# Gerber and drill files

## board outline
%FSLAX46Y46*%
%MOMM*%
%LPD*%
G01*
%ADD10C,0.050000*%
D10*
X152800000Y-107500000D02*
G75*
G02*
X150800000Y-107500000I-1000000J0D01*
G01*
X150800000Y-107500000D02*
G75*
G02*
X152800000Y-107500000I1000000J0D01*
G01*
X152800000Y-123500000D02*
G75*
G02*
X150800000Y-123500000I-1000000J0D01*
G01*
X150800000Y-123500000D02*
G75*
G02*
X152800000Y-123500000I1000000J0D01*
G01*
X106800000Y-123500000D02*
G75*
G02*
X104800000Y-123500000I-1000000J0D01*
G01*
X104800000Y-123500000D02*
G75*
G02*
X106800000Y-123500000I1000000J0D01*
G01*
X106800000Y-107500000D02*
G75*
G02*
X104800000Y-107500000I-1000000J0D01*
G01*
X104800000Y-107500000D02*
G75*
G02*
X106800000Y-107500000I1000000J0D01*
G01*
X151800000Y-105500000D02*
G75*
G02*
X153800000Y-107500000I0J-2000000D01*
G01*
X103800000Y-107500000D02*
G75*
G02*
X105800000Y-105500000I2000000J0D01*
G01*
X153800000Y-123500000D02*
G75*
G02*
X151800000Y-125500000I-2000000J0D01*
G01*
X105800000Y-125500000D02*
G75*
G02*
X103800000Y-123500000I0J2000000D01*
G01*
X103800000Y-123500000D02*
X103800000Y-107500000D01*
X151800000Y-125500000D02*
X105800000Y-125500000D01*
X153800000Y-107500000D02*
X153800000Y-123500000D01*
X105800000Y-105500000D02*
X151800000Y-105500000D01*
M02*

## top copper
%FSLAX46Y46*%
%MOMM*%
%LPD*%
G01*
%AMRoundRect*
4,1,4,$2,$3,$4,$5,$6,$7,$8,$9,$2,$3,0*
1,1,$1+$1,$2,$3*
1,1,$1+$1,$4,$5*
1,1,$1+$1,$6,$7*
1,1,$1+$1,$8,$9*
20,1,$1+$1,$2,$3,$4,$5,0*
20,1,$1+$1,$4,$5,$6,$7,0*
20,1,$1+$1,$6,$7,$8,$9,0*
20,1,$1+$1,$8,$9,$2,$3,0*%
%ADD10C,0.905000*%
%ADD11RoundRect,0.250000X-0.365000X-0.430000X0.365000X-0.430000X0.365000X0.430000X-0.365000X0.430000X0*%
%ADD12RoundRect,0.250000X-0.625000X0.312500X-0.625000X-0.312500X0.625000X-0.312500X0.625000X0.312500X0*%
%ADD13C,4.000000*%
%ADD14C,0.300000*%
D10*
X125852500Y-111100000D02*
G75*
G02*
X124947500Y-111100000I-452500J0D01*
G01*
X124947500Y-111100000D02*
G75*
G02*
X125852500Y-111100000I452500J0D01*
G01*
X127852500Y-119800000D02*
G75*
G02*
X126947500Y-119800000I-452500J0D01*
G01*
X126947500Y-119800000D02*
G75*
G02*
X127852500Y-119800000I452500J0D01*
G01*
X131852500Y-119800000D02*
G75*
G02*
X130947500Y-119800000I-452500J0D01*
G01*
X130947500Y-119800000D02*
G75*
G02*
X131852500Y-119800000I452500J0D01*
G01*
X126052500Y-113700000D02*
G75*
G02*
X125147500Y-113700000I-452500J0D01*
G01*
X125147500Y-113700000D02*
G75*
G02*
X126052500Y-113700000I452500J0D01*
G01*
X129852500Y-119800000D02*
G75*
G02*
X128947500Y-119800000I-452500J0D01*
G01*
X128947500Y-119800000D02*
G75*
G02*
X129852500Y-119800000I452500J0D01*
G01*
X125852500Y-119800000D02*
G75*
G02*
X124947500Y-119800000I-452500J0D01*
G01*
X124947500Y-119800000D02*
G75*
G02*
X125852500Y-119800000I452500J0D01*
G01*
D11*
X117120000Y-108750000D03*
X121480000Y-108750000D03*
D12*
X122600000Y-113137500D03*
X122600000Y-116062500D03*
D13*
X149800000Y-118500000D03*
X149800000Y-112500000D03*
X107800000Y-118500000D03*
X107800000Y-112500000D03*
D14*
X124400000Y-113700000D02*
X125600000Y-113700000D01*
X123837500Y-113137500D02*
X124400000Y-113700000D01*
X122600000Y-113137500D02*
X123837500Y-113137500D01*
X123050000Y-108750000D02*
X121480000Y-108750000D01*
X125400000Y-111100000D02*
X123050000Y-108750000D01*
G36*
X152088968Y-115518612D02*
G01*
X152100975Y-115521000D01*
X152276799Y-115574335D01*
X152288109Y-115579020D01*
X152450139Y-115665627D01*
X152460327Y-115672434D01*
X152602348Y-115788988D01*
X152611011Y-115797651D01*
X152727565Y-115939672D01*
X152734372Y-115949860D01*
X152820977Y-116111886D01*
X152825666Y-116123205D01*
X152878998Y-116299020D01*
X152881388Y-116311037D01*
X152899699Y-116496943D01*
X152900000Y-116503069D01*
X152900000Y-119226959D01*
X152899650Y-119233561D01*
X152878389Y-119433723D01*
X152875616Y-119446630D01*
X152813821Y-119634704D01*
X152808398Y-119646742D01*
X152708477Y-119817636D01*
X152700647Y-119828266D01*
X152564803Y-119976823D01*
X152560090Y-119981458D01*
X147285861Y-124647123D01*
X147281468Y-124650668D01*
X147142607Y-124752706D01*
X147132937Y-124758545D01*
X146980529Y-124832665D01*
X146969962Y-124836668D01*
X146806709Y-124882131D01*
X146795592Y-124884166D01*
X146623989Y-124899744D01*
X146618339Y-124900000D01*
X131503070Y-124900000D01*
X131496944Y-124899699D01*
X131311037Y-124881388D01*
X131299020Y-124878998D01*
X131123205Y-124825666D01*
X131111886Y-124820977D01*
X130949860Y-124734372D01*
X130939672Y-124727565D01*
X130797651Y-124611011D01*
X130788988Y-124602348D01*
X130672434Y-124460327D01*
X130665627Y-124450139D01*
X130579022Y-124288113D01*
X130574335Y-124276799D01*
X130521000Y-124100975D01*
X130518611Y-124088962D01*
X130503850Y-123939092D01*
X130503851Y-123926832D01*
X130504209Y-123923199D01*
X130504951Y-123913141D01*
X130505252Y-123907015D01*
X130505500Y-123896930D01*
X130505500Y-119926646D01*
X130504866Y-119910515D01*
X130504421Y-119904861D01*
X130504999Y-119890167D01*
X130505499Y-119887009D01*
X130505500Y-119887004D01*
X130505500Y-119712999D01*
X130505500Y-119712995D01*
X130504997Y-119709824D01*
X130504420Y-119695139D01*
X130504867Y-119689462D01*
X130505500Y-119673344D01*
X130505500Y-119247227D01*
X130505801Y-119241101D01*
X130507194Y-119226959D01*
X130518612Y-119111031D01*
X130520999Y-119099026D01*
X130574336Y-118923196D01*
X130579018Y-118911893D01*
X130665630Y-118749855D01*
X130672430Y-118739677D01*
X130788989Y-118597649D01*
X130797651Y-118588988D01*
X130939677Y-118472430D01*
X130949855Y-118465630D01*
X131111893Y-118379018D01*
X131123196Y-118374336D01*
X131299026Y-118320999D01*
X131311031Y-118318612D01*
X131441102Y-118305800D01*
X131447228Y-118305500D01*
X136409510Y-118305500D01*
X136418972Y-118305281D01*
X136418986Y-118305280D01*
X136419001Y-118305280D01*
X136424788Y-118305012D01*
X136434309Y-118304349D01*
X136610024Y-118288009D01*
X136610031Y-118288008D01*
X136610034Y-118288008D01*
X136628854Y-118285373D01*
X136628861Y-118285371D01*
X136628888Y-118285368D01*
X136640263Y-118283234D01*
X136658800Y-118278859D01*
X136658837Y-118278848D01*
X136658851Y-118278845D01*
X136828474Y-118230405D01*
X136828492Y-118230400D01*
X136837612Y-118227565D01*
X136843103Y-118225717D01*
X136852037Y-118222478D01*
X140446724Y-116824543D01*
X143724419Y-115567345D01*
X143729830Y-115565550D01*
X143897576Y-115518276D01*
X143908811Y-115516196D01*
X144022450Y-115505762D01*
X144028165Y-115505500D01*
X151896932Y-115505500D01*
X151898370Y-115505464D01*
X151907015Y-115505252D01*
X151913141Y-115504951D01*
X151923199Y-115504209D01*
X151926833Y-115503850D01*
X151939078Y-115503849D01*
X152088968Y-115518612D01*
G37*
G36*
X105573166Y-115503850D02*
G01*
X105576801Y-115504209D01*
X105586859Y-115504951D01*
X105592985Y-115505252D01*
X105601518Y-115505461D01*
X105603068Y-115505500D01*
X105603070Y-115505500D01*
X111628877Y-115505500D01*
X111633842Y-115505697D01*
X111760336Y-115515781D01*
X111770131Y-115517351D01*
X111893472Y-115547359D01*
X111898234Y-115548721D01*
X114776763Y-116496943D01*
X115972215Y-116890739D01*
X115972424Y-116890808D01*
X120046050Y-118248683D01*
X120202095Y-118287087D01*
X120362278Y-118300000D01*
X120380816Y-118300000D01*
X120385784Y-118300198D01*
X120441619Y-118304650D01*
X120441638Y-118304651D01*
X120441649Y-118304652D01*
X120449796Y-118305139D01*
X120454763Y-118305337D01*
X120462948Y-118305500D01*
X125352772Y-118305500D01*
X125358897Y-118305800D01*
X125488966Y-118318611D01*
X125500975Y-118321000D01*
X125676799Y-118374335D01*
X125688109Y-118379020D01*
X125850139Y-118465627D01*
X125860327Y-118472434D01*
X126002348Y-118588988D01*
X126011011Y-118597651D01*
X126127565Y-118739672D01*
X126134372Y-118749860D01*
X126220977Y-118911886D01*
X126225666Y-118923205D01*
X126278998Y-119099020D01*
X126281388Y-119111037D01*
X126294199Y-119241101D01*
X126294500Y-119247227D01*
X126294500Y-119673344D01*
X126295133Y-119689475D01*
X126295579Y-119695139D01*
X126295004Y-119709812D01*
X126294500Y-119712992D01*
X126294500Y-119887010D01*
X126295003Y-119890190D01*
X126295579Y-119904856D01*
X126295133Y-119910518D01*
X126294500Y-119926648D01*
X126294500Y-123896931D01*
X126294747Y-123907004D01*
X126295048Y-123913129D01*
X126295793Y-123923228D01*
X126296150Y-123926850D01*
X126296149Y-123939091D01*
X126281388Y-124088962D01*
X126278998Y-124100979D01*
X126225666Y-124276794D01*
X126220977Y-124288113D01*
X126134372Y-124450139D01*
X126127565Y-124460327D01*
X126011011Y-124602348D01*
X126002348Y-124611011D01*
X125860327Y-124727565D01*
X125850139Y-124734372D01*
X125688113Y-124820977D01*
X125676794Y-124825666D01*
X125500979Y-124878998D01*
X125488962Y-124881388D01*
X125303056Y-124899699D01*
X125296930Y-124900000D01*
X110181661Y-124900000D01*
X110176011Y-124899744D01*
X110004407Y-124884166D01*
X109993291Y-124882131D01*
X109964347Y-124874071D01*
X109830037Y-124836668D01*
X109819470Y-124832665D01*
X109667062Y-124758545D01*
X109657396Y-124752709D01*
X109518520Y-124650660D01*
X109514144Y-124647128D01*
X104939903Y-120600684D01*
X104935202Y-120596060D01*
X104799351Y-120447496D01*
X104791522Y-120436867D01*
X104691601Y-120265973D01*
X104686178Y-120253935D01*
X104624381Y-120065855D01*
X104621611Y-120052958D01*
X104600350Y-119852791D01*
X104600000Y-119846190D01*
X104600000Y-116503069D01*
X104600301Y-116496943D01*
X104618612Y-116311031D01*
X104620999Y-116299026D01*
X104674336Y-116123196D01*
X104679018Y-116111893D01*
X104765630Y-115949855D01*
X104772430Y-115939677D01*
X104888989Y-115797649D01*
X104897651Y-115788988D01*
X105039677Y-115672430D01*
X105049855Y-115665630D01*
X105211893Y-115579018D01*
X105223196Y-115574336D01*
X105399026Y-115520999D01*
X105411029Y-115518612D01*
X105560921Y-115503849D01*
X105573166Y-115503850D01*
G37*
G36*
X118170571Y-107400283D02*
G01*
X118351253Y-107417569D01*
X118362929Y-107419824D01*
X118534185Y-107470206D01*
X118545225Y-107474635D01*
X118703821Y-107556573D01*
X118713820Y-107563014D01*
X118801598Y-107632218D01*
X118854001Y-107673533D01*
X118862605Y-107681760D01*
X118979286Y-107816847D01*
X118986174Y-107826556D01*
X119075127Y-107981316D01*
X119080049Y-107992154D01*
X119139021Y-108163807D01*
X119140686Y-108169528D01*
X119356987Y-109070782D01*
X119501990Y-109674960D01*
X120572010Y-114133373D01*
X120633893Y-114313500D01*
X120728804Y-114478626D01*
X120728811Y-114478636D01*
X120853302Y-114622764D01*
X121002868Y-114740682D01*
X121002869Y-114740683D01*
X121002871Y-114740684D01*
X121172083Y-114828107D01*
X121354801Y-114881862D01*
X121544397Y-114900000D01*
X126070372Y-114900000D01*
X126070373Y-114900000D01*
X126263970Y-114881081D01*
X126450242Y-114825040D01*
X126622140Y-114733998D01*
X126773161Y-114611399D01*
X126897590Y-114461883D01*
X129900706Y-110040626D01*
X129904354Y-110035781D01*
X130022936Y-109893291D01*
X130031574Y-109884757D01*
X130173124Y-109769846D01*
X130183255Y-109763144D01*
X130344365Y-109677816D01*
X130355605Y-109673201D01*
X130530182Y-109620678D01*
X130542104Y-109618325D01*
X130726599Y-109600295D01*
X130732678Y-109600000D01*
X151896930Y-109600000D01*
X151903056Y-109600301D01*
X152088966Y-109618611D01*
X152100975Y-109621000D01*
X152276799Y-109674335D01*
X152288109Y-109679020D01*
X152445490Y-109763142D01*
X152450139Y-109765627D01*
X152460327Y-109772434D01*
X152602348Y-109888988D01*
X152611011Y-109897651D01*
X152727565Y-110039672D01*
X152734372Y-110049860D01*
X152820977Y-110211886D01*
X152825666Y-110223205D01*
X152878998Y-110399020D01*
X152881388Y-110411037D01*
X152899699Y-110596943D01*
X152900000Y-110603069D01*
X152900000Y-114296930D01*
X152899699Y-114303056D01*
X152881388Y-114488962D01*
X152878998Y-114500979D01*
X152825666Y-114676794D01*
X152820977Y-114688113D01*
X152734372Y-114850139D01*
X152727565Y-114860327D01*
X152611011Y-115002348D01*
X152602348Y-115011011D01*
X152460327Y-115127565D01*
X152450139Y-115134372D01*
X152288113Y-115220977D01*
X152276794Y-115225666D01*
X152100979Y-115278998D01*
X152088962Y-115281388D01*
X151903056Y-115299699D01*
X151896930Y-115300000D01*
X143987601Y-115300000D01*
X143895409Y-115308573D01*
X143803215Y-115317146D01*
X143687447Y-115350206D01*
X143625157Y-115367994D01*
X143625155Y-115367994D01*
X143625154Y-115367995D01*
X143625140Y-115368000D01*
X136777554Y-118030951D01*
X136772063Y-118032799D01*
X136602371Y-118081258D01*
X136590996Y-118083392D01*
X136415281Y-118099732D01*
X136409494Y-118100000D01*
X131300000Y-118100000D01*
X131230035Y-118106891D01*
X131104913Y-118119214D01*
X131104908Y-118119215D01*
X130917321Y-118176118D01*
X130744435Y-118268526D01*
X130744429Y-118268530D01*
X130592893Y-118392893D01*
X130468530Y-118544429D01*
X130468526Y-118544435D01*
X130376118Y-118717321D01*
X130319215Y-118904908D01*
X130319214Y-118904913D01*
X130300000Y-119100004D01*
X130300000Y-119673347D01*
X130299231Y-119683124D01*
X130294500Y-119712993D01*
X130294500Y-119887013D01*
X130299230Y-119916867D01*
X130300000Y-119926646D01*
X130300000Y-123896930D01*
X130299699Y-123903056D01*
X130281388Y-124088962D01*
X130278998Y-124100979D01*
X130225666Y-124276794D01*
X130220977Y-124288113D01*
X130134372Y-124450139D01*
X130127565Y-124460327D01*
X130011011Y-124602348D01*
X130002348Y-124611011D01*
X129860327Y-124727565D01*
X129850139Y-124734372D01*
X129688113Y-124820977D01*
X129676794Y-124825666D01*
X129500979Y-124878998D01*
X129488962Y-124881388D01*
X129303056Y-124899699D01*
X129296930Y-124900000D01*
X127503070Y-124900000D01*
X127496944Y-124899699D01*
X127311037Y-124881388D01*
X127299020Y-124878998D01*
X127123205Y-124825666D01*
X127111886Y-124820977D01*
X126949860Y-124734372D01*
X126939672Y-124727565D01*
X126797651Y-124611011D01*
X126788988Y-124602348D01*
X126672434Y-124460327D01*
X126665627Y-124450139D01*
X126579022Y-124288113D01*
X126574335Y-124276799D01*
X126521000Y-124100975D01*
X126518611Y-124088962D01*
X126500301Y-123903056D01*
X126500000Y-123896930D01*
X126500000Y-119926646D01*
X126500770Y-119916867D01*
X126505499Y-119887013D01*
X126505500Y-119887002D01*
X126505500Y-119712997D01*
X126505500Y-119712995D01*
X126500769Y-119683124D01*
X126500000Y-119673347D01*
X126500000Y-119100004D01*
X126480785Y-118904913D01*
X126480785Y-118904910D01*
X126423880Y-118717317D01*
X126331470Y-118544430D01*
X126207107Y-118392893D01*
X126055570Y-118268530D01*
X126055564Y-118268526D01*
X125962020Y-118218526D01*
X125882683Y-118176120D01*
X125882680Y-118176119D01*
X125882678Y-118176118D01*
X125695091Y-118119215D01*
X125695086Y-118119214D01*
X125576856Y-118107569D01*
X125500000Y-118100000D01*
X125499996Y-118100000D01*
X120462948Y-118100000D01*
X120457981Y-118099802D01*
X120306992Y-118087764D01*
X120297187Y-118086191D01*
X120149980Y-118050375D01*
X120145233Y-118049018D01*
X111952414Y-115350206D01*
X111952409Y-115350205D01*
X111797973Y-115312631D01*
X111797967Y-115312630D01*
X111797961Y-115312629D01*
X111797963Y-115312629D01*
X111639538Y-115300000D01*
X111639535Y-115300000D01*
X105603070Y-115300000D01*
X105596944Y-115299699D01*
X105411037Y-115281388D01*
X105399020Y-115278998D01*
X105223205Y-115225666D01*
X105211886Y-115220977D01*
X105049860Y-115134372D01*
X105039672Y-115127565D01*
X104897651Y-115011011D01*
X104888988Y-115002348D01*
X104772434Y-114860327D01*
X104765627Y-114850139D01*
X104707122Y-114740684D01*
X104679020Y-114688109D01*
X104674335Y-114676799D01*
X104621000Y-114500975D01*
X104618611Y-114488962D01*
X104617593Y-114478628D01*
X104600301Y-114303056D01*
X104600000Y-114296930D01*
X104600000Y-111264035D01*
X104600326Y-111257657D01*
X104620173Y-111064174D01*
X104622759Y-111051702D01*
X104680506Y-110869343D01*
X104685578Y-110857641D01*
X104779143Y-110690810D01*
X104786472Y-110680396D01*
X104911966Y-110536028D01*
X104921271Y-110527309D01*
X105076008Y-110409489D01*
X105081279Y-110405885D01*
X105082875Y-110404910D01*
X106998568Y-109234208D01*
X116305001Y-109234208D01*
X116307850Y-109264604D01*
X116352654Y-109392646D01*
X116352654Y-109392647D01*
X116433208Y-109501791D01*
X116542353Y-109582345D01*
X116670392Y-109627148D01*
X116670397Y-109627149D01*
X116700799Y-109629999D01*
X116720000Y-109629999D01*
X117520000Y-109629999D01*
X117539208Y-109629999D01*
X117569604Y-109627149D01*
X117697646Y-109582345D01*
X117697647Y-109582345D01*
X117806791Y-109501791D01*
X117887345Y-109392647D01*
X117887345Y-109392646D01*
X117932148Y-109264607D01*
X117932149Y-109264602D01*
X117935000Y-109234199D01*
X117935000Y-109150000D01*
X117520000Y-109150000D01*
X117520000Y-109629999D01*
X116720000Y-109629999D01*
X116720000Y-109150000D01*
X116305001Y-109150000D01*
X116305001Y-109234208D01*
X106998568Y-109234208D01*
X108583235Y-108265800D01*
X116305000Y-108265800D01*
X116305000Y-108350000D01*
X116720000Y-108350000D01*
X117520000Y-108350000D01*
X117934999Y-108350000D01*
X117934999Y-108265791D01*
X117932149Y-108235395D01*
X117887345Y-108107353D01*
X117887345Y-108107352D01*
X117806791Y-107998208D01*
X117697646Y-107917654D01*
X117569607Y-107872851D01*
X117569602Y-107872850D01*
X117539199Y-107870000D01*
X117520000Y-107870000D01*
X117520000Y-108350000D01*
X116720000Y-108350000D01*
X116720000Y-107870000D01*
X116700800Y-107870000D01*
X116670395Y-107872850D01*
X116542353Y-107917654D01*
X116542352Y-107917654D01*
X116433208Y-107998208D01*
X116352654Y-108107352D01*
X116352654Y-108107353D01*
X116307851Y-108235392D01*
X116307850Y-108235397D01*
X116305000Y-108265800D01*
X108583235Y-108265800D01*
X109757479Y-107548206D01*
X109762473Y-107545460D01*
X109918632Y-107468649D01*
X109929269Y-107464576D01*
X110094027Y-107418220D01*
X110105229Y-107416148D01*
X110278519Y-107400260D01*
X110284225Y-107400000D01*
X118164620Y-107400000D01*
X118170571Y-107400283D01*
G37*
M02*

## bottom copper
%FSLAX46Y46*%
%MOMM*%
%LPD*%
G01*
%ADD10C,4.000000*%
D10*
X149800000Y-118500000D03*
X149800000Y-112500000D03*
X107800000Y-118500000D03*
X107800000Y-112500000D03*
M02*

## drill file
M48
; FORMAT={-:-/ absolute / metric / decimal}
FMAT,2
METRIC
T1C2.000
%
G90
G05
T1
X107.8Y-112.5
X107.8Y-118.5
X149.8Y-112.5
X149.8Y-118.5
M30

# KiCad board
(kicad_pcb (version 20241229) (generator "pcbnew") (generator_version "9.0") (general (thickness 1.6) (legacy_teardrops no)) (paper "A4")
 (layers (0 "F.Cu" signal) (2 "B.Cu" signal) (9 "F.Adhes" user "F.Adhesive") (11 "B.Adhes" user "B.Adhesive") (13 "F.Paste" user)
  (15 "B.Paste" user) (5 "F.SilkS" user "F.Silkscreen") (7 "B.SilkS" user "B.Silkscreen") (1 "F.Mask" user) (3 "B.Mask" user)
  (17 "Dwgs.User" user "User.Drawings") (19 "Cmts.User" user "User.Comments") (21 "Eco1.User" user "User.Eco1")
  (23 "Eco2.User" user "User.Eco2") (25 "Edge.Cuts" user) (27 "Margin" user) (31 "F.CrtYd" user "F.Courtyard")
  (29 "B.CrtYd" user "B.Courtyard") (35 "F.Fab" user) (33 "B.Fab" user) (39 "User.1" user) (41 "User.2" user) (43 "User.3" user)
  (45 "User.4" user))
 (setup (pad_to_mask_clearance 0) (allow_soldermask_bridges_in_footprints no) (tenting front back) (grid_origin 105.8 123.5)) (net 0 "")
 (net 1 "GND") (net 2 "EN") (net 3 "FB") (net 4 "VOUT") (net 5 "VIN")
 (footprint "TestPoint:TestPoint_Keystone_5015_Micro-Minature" (layer "F.Cu") (at 131.4 119.8)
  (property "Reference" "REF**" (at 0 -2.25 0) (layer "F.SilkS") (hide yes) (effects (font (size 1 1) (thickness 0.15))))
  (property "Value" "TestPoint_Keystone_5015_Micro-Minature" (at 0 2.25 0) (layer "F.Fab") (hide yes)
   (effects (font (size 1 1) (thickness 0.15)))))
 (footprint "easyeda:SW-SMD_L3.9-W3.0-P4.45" (layer "F.Cu") (at 119.3 108.75)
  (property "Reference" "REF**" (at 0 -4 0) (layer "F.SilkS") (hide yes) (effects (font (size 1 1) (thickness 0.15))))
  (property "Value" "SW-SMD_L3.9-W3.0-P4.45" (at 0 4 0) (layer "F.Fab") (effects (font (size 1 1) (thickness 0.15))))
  (pad "1" smd roundrect (at -2.18 0) (size 1.23 1.36) (layers "F.Cu" "F.Mask" "F.Paste") (roundrect_rratio 0.2032520325) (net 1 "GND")
   (zone_connect 1) (thermal_bridge_width 0.8) (thermal_gap 0.2))
  (pad "2" smd roundrect (at 2.18 0) (size 1.23 1.36) (layers "F.Cu" "F.Mask" "F.Paste") (roundrect_rratio 0.2032520325) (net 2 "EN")))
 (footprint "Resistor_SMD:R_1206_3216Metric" (layer "F.Cu") (at 122.6 114.6 -90)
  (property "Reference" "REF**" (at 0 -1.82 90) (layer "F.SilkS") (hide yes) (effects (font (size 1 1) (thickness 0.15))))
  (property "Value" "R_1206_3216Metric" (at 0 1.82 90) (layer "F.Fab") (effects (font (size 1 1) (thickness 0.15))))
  (pad "1" smd roundrect (at -1.4625 0 270) (size 1.125 1.75) (layers "F.Cu" "F.Mask" "F.Paste") (roundrect_rratio 0.222222) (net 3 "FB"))
  (pad "2" smd roundrect (at 1.4625 0 270) (size 1.125 1.75) (layers "F.Cu" "F.Mask" "F.Paste") (roundrect_rratio 0.222222) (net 1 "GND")))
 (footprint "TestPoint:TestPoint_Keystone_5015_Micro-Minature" (layer "F.Cu") (at 125.4 119.8)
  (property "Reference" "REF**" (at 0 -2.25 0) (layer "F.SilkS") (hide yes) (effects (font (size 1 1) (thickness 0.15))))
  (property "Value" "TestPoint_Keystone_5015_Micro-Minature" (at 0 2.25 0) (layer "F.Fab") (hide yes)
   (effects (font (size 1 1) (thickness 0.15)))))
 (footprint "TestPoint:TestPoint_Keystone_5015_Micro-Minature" (layer "F.Cu") (at 128.5 115.5)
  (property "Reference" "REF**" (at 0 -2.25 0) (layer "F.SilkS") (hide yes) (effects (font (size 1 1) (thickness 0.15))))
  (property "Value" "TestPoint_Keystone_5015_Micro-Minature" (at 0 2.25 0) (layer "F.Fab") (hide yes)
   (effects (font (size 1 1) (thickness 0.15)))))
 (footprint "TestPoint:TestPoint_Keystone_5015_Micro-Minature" (layer "F.Cu") (at 125.6 113.7)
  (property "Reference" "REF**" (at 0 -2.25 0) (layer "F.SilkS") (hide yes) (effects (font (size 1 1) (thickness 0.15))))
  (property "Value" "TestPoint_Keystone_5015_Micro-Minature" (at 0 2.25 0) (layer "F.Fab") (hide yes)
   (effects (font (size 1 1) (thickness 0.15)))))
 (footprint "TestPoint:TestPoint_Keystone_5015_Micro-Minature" (layer "F.Cu") (at 125.4 111.1)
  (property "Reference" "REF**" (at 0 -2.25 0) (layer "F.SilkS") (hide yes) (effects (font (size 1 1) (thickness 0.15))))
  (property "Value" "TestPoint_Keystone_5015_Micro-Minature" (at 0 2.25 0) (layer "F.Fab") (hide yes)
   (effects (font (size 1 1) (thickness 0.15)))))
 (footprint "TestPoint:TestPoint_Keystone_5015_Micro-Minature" (layer "F.Cu") (at 129.4 119.8)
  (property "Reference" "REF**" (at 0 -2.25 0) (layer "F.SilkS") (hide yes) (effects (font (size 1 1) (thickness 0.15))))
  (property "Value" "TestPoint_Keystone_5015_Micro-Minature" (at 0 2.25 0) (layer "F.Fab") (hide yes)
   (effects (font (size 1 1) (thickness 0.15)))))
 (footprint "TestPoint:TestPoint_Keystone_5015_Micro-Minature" (layer "F.Cu") (at 127.4 119.8)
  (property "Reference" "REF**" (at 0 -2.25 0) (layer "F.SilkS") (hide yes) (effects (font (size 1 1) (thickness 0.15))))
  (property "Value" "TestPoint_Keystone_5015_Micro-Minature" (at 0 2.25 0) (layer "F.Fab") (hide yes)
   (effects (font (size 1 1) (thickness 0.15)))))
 (gr_circle (center 125.4 111.1) (end 126.3 111.1) (stroke (width 0.01) (type default)) (fill yes) (layer "F.Cu") (net 2))
 (gr_circle (center 127.4 119.8) (end 128.3 119.8) (stroke (width 0.01) (type default)) (fill yes) (layer "F.Cu") (net 1))
 (gr_circle (center 131.4 119.8) (end 132.3 119.8) (stroke (width 0.01) (type default)) (fill yes) (layer "F.Cu") (net 4))
 (gr_circle (center 125.6 113.7) (end 126.5 113.7) (stroke (width 0.01) (type solid)) (fill yes) (layer "F.Cu") (net 3))
 (gr_circle (center 129.4 119.8) (end 130.3 119.8) (stroke (width 0.01) (type default)) (fill yes) (layer "F.Cu") (net 1))
 (gr_circle (center 125.4 119.8) (end 126.3 119.8) (stroke (width 0.01) (type default)) (fill yes) (layer "F.Cu") (net 5))
 (gr_circle (center 151.8 123.5) (end 151.8 122.5) (stroke (width 0.05) (type default)) (fill no) (layer "Edge.Cuts"))
 (gr_circle (center 151.8 107.5) (end 151.8 108.5) (stroke (width 0.05) (type default)) (fill no) (layer "Edge.Cuts"))
 (gr_line (start 105.8 105.5) (end 151.8 105.5) (stroke (width 0.05) (type default)) (layer "Edge.Cuts"))
 (gr_line (start 103.8 123.5) (end 103.8 107.5) (stroke (width 0.05) (type default)) (layer "Edge.Cuts"))
 (gr_circle (center 105.8 123.5) (end 105.8 122.5) (stroke (width 0.05) (type default)) (fill no) (layer "Edge.Cuts"))
 (gr_arc (start 105.8 125.5) (mid 104.385786 124.914214) (end 103.8 123.5) (stroke (width 0.05) (type default)) (layer "Edge.Cuts"))
 (gr_line (start 151.8 125.5) (end 105.8 125.5) (stroke (width 0.05) (type default)) (layer "Edge.Cuts"))
 (gr_arc (start 153.8 123.5) (mid 153.214214 124.914214) (end 151.8 125.5) (stroke (width 0.05) (type default)) (layer "Edge.Cuts"))
 (gr_circle (center 105.8 107.5) (end 105.8 106.5) (stroke (width 0.05) (type default)) (fill no) (layer "Edge.Cuts"))
 (gr_arc (start 103.8 107.5) (mid 104.385786 106.085786) (end 105.8 105.5) (stroke (width 0.05) (type default)) (layer "Edge.Cuts"))
 (gr_line (start 153.8 107.5) (end 153.8 123.5) (stroke (width 0.05) (type default)) (layer "Edge.Cuts"))
 (gr_arc (start 151.8 105.5) (mid 153.214214 106.085786) (end 153.8 107.5) (stroke (width 0.05) (type default)) (layer "Edge.Cuts"))
 (via (at 149.8 118.5) (size 4) (drill 2) (layers "F.Cu" "B.Cu") (tenting none) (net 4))
 (via (at 149.8 112.5) (size 4) (drill 2) (layers "F.Cu" "B.Cu") (tenting none) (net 1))
 (via (at 107.8 112.5) (size 4) (drill 2) (layers "F.Cu" "B.Cu") (tenting none) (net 1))
 (via (at 107.8 118.5) (size 4) (drill 2) (layers "F.Cu" "B.Cu") (tenting none) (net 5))
 (segment (start 125.4 111.1) (end 123.05 108.75) (width 0.3) (layer "F.Cu") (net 2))
 (segment (start 123.05 108.75) (end 121.48 108.75) (width 0.3) (layer "F.Cu") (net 2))
 (segment (start 122.6 113.1375) (end 123.8375 113.1375) (width 0.3) (layer "F.Cu") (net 3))
 (segment (start 124.4 113.7) (end 125.6 113.7) (width 0.3) (layer "F.Cu") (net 3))
 (segment (start 123.8375 113.1375) (end 124.4 113.7) (width 0.3) (layer "F.Cu") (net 3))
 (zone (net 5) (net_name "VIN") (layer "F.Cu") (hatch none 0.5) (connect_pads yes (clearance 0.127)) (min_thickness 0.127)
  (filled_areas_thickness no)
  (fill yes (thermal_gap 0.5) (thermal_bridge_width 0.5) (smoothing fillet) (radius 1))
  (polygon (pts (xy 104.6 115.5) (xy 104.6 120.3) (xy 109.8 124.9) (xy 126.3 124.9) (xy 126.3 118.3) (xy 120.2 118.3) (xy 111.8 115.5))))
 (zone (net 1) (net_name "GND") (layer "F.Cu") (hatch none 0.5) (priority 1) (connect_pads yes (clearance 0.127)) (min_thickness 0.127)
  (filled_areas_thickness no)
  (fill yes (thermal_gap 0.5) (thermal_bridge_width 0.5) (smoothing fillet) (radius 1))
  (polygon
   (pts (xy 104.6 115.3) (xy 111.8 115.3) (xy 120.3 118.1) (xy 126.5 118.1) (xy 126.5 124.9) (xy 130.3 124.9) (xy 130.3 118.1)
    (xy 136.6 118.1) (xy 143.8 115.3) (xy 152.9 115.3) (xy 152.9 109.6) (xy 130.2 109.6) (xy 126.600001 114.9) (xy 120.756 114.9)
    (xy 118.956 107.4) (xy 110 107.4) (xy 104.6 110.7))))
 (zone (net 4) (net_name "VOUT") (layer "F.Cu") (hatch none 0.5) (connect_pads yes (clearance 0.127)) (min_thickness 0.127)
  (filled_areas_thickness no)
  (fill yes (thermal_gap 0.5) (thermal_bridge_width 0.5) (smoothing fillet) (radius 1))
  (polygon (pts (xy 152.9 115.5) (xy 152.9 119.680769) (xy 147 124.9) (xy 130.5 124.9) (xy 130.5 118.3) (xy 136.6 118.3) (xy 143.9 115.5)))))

